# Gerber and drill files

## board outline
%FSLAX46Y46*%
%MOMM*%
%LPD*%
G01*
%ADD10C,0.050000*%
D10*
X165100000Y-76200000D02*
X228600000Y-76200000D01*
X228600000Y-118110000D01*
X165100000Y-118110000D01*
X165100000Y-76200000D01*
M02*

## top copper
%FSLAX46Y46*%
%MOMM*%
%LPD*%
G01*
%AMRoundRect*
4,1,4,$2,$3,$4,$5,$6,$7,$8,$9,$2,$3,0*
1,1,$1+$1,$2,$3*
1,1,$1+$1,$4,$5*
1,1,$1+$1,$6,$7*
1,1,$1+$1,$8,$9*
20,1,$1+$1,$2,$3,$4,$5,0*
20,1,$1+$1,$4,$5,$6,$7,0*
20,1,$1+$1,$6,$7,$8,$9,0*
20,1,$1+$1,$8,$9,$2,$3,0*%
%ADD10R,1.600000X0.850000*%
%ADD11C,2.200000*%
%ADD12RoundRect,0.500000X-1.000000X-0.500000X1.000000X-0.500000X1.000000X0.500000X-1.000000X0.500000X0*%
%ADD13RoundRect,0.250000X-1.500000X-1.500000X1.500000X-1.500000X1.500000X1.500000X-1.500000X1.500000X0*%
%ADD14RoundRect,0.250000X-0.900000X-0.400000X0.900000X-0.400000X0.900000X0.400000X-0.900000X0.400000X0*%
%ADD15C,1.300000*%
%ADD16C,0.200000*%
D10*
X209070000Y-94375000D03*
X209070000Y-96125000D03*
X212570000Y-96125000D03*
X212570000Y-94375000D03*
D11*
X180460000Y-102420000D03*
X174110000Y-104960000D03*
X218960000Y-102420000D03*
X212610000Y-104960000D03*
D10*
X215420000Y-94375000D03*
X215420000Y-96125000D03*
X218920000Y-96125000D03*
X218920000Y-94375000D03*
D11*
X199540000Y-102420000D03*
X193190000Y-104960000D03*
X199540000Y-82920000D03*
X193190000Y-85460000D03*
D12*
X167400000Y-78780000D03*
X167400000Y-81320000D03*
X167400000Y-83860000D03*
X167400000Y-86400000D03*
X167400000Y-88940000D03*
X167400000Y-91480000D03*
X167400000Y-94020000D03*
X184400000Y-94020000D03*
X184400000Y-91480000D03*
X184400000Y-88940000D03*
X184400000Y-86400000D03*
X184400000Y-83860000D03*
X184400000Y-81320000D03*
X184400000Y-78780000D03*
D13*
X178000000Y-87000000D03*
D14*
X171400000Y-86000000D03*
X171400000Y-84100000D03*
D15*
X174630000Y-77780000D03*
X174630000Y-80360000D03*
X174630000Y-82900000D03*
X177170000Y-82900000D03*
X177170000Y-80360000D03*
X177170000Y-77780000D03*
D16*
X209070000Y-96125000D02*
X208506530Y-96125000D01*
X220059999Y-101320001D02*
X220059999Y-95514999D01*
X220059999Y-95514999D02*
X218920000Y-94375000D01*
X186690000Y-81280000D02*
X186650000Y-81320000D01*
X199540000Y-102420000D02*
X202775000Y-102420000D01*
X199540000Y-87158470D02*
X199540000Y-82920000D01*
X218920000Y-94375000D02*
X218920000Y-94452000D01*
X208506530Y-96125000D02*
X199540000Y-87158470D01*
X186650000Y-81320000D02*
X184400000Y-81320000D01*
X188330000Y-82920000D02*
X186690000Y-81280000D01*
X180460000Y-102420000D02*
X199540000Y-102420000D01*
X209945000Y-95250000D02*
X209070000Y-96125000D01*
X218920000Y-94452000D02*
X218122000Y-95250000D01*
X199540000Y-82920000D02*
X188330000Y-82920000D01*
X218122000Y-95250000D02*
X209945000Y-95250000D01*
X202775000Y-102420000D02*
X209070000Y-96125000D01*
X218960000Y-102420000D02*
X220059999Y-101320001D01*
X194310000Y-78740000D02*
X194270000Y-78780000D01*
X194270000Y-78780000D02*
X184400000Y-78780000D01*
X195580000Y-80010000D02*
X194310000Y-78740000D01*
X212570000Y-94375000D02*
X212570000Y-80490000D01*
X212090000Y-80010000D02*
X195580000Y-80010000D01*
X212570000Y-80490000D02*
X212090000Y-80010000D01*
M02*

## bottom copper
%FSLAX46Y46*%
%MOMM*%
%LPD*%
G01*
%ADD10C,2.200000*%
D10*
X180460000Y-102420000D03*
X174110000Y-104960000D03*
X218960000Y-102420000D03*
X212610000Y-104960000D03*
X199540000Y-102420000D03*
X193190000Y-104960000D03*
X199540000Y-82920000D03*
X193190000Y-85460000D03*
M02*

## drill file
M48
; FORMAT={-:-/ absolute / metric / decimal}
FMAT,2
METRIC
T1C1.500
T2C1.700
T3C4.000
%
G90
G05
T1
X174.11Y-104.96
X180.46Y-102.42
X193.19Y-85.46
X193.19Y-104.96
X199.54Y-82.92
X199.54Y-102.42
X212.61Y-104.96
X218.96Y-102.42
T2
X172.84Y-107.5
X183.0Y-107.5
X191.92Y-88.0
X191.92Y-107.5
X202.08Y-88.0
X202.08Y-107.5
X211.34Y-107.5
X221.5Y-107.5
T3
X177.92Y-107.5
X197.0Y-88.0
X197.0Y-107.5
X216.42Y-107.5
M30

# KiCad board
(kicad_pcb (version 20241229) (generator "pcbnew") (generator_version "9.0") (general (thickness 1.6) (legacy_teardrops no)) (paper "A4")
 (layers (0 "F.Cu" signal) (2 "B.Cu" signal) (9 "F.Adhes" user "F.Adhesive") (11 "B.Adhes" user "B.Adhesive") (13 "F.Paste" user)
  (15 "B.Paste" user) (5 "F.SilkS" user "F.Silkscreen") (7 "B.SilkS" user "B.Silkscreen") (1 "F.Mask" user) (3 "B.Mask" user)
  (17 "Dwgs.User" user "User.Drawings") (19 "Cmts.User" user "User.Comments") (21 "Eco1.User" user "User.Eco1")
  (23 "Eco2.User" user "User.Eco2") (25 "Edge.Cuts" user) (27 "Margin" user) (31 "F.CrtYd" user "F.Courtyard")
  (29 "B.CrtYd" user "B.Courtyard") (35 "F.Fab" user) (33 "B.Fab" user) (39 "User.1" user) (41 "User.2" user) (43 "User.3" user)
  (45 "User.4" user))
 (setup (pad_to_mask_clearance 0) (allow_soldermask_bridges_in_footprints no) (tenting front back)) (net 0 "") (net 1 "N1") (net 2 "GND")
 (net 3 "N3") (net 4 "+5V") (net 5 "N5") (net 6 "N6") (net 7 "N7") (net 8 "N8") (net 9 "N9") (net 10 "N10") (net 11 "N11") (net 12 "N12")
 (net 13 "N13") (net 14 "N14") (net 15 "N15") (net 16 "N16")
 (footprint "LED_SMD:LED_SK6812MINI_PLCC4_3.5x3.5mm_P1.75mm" (layer "F.Cu") (at 210.82 95.25)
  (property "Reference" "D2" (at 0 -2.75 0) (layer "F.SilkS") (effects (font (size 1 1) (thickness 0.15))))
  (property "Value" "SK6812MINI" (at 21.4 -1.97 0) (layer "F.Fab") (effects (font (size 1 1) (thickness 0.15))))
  (pad "1" smd rect (at -1.75 -0.875) (size 1.6 0.85) (layers "F.Cu" "F.Mask" "F.Paste") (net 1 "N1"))
  (pad "2" smd rect (at -1.75 0.875) (size 1.6 0.85) (layers "F.Cu" "F.Mask" "F.Paste") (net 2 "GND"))
  (pad "3" smd rect (at 1.75 0.875) (size 1.6 0.85) (layers "F.Cu" "F.Mask" "F.Paste") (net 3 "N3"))
  (pad "4" smd rect (at 1.75 -0.875) (size 1.6 0.85) (layers "F.Cu" "F.Mask" "F.Paste") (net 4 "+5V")))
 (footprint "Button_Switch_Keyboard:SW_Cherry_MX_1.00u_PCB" (layer "F.Cu") (at 180.46 102.42)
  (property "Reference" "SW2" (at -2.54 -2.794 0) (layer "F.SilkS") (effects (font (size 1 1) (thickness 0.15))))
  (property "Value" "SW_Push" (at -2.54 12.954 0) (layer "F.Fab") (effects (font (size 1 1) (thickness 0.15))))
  (pad "" np_thru_hole circle (at -7.62 5.08) (size 1.7 1.7) (drill 1.7) (layers "*.Cu" "*.Mask"))
  (pad "" np_thru_hole circle (at -2.54 5.08) (size 4 4) (drill 4) (layers "*.Cu" "*.Mask"))
  (pad "" np_thru_hole circle (at 2.54 5.08) (size 1.7 1.7) (drill 1.7) (layers "*.Cu" "*.Mask"))
  (pad "1" thru_hole circle (at 0 0) (size 2.2 2.2) (drill 1.5) (layers "*.Cu" "*.Mask") (remove_unused_layers no) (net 2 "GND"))
  (pad "2" thru_hole circle (at -6.35 2.54) (size 2.2 2.2) (drill 1.5) (layers "*.Cu" "*.Mask") (remove_unused_layers no) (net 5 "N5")))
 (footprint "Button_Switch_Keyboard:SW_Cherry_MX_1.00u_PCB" (layer "F.Cu") (at 218.96 102.42)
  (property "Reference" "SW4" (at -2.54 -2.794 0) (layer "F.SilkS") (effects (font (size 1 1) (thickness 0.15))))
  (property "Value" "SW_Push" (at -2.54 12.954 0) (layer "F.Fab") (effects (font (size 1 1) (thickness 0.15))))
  (pad "" np_thru_hole circle (at -7.62 5.08) (size 1.7 1.7) (drill 1.7) (layers "*.Cu" "*.Mask"))
  (pad "" np_thru_hole circle (at -2.54 5.08) (size 4 4) (drill 4) (layers "*.Cu" "*.Mask"))
  (pad "" np_thru_hole circle (at 2.54 5.08) (size 1.7 1.7) (drill 1.7) (layers "*.Cu" "*.Mask"))
  (pad "1" thru_hole circle (at 0 0) (size 2.2 2.2) (drill 1.5) (layers "*.Cu" "*.Mask") (remove_unused_layers no) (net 2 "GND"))
  (pad "2" thru_hole circle (at -6.35 2.54) (size 2.2 2.2) (drill 1.5) (layers "*.Cu" "*.Mask") (remove_unused_layers no) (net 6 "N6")))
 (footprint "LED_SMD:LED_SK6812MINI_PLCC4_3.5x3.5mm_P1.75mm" (layer "F.Cu") (at 217.17 95.25)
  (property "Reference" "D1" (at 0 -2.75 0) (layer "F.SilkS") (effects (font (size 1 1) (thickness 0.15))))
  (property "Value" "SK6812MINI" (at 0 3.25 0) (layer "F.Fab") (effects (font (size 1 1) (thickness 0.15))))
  (pad "1" smd rect (at -1.75 -0.875) (size 1.6 0.85) (layers "F.Cu" "F.Mask" "F.Paste") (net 3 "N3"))
  (pad "2" smd rect (at -1.75 0.875) (size 1.6 0.85) (layers "F.Cu" "F.Mask" "F.Paste") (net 4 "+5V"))
  (pad "3" smd rect (at 1.75 0.875) (size 1.6 0.85) (layers "F.Cu" "F.Mask" "F.Paste") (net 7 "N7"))
  (pad "4" smd rect (at 1.75 -0.875) (size 1.6 0.85) (layers "F.Cu" "F.Mask" "F.Paste") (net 2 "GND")))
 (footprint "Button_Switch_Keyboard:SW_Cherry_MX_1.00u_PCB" (layer "F.Cu") (at 199.54 102.42)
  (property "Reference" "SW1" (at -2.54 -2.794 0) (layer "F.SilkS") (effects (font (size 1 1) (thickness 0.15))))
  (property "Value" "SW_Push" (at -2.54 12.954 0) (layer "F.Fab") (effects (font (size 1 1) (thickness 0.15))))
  (pad "" np_thru_hole circle (at -7.62 5.08) (size 1.7 1.7) (drill 1.7) (layers "*.Cu" "*.Mask"))
  (pad "" np_thru_hole circle (at -2.54 5.08) (size 4 4) (drill 4) (layers "*.Cu" "*.Mask"))
  (pad "" np_thru_hole circle (at 2.54 5.08) (size 1.7 1.7) (drill 1.7) (layers "*.Cu" "*.Mask"))
  (pad "1" thru_hole circle (at 0 0) (size 2.2 2.2) (drill 1.5) (layers "*.Cu" "*.Mask") (remove_unused_layers no) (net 2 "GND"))
  (pad "2" thru_hole circle (at -6.35 2.54) (size 2.2 2.2) (drill 1.5) (layers "*.Cu" "*.Mask") (remove_unused_layers no) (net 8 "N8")))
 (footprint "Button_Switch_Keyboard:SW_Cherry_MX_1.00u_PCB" (layer "F.Cu") (at 199.54 82.92)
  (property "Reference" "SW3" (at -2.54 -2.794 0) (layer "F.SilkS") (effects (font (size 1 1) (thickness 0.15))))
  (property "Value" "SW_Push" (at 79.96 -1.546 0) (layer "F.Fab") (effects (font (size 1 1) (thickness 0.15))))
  (pad "" np_thru_hole circle (at -7.62 5.08) (size 1.7 1.7) (drill 1.7) (layers "*.Cu" "*.Mask"))
  (pad "" np_thru_hole circle (at -2.54 5.08) (size 4 4) (drill 4) (layers "*.Cu" "*.Mask"))
  (pad "" np_thru_hole circle (at 2.54 5.08) (size 1.7 1.7) (drill 1.7) (layers "*.Cu" "*.Mask"))
  (pad "1" thru_hole circle (at 0 0) (size 2.2 2.2) (drill 1.5) (layers "*.Cu" "*.Mask") (remove_unused_layers no) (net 2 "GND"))
  (pad "2" thru_hole circle (at -6.35 2.54) (size 2.2 2.2) (drill 1.5) (layers "*.Cu" "*.Mask") (remove_unused_layers no) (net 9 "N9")))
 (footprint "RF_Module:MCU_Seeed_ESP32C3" (layer "F.Cu") (at 175.9 86.4)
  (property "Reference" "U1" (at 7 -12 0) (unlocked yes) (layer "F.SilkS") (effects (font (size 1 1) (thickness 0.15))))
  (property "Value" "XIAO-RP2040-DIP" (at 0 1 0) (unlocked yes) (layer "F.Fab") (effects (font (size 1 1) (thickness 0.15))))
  (pad "" smd roundrect (at 1.1 -0.4) (size 1.5 1.5) (layers "F.Paste") (roundrect_rratio 0.1666666667))
  (pad "" smd roundrect (at 1.1 1.6) (size 1.5 1.5) (layers "F.Paste") (roundrect_rratio 0.1666666667))
  (pad "" smd roundrect (at 3.1 -0.4) (size 1.5 1.5) (layers "F.Paste") (roundrect_rratio 0.1666666667))
  (pad "" smd roundrect (at 3.1 1.6) (size 1.5 1.5) (layers "F.Paste") (roundrect_rratio 0.1666666667))
  (pad "1" smd roundrect (at -8.5 -7.62) (size 3 2) (layers "F.Cu" "F.Mask" "F.Paste") (roundrect_rratio 0.25) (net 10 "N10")
   (thermal_bridge_angle 45))
  (pad "2" smd roundrect (at -8.5 -5.08) (size 3 2) (layers "F.Cu" "F.Mask" "F.Paste") (roundrect_rratio 0.25) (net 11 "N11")
   (thermal_bridge_angle 45))
  (pad "3" smd roundrect (at -8.5 -2.54) (size 3 2) (layers "F.Cu" "F.Mask" "F.Paste") (roundrect_rratio 0.25) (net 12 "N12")
   (thermal_bridge_angle 45))
  (pad "4" smd roundrect (at -8.5 0) (size 3 2) (layers "F.Cu" "F.Mask" "F.Paste") (roundrect_rratio 0.25) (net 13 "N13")
   (thermal_bridge_angle 45))
  (pad "5" smd roundrect (at -8.5 2.54) (size 3 2) (layers "F.Cu" "F.Mask" "F.Paste") (roundrect_rratio 0.25) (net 7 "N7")
   (thermal_bridge_angle 45))
  (pad "6" smd roundrect (at -8.5 5.08) (size 3 2) (layers "F.Cu" "F.Mask" "F.Paste") (roundrect_rratio 0.25) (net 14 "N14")
   (thermal_bridge_angle 45))
  (pad "7" smd roundrect (at -8.5 7.62) (size 3 2) (layers "F.Cu" "F.Mask" "F.Paste") (roundrect_rratio 0.25) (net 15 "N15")
   (thermal_bridge_angle 45))
  (pad "8" smd roundrect (at 8.5 7.62) (size 3 2) (layers "F.Cu" "F.Mask" "F.Paste") (roundrect_rratio 0.25) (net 8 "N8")
   (thermal_bridge_angle 45))
  (pad "9" smd roundrect (at 8.5 5.08) (size 3 2) (layers "F.Cu" "F.Mask" "F.Paste") (roundrect_rratio 0.25) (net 5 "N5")
   (thermal_bridge_angle 45))
  (pad "10" smd roundrect (at 8.5 2.54) (size 3 2) (layers "F.Cu" "F.Mask" "F.Paste") (roundrect_rratio 0.25) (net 9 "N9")
   (thermal_bridge_angle 45))
  (pad "11" smd roundrect (at 8.5 0) (size 3 2) (layers "F.Cu" "F.Mask" "F.Paste") (roundrect_rratio 0.25) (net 6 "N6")
   (thermal_bridge_angle 45))
  (pad "12" smd roundrect (at 8.5 -2.54) (size 3 2) (layers "F.Cu" "F.Mask" "F.Paste") (roundrect_rratio 0.25) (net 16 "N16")
   (thermal_bridge_angle 45))
  (pad "13" smd roundrect (at 8.5 -5.08) (size 3 2) (layers "F.Cu" "F.Mask" "F.Paste") (roundrect_rratio 0.25) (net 2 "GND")
   (thermal_bridge_angle 45))
  (pad "14" smd roundrect (at 8.5 -7.62) (size 3 2) (layers "F.Cu" "F.Mask" "F.Paste") (roundrect_rratio 0.25) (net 4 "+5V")
   (thermal_bridge_angle 45))
  (pad "15" smd roundrect (at 2.1 0.6) (size 3.5 3.5) (layers "F.Cu" "F.Mask") (roundrect_rratio 0.07142857143))
  (pad "16" smd roundrect (at -4.5 -0.4) (size 2.3 1.3) (layers "F.Cu" "F.Mask" "F.Paste") (roundrect_rratio 0.1923076923))
  (pad "17" smd roundrect (at -4.5 -2.3) (size 2.3 1.3) (layers "F.Cu" "F.Mask" "F.Paste") (roundrect_rratio 0.1923076923))
  (pad "18" smd circle (at -1.27 -8.62) (size 1.3 1.3) (layers "F.Cu" "F.Mask" "F.Paste"))
  (pad "19" smd circle (at -1.27 -6.04) (size 1.3 1.3) (layers "F.Cu" "F.Mask" "F.Paste"))
  (pad "20" smd circle (at -1.27 -3.5) (size 1.3 1.3) (layers "F.Cu" "F.Mask" "F.Paste"))
  (pad "21" smd circle (at 1.27 -3.5) (size 1.3 1.3) (layers "F.Cu" "F.Mask" "F.Paste"))
  (pad "22" smd circle (at 1.27 -6.04) (size 1.3 1.3) (layers "F.Cu" "F.Mask" "F.Paste"))
  (pad "23" smd circle (at 1.27 -8.62) (size 1.3 1.3) (layers "F.Cu" "F.Mask" "F.Paste")))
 (gr_rect (start 165.1 76.2) (end 228.6 118.11) (stroke (width 0.05) (type default)) (fill no) (layer "Edge.Cuts"))
 (segment (start 209.07 96.125) (end 208.50653 96.125) (width 0.2) (layer "F.Cu") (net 2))
 (segment (start 220.059999 101.320001) (end 220.059999 95.514999) (width 0.2) (layer "F.Cu") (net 2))
 (segment (start 220.059999 95.514999) (end 218.92 94.375) (width 0.2) (layer "F.Cu") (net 2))
 (segment (start 186.69 81.28) (end 186.65 81.32) (width 0.2) (layer "F.Cu") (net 2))
 (segment (start 199.54 102.42) (end 202.775 102.42) (width 0.2) (layer "F.Cu") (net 2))
 (segment (start 199.54 87.15847) (end 199.54 82.92) (width 0.2) (layer "F.Cu") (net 2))
 (segment (start 218.92 94.375) (end 218.92 94.452) (width 0.2) (layer "F.Cu") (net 2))
 (segment (start 208.50653 96.125) (end 199.54 87.15847) (width 0.2) (layer "F.Cu") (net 2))
 (segment (start 186.65 81.32) (end 184.4 81.32) (width 0.2) (layer "F.Cu") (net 2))
 (segment (start 188.33 82.92) (end 186.69 81.28) (width 0.2) (layer "F.Cu") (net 2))
 (segment (start 180.46 102.42) (end 199.54 102.42) (width 0.2) (layer "F.Cu") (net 2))
 (segment (start 209.945 95.25) (end 209.07 96.125) (width 0.2) (layer "F.Cu") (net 2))
 (segment (start 218.92 94.452) (end 218.122 95.25) (width 0.2) (layer "F.Cu") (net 2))
 (segment (start 199.54 82.92) (end 188.33 82.92) (width 0.2) (layer "F.Cu") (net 2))
 (segment (start 218.122 95.25) (end 209.945 95.25) (width 0.2) (layer "F.Cu") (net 2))
 (segment (start 202.775 102.42) (end 209.07 96.125) (width 0.2) (layer "F.Cu") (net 2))
 (segment (start 218.96 102.42) (end 220.059999 101.320001) (width 0.2) (layer "F.Cu") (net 2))
 (segment (start 194.31 78.74) (end 194.27 78.78) (width 0.2) (layer "F.Cu") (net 4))
 (segment (start 194.27 78.78) (end 184.4 78.78) (width 0.2) (layer "F.Cu") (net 4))
 (segment (start 195.58 80.01) (end 194.31 78.74) (width 0.2) (layer "F.Cu") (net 4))
 (segment (start 212.57 94.375) (end 212.57 80.49) (width 0.2) (layer "F.Cu") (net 4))
 (segment (start 212.09 80.01) (end 195.58 80.01) (width 0.2) (layer "F.Cu") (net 4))
 (segment (start 212.57 80.49) (end 212.09 80.01) (width 0.2) (layer "F.Cu") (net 4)))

